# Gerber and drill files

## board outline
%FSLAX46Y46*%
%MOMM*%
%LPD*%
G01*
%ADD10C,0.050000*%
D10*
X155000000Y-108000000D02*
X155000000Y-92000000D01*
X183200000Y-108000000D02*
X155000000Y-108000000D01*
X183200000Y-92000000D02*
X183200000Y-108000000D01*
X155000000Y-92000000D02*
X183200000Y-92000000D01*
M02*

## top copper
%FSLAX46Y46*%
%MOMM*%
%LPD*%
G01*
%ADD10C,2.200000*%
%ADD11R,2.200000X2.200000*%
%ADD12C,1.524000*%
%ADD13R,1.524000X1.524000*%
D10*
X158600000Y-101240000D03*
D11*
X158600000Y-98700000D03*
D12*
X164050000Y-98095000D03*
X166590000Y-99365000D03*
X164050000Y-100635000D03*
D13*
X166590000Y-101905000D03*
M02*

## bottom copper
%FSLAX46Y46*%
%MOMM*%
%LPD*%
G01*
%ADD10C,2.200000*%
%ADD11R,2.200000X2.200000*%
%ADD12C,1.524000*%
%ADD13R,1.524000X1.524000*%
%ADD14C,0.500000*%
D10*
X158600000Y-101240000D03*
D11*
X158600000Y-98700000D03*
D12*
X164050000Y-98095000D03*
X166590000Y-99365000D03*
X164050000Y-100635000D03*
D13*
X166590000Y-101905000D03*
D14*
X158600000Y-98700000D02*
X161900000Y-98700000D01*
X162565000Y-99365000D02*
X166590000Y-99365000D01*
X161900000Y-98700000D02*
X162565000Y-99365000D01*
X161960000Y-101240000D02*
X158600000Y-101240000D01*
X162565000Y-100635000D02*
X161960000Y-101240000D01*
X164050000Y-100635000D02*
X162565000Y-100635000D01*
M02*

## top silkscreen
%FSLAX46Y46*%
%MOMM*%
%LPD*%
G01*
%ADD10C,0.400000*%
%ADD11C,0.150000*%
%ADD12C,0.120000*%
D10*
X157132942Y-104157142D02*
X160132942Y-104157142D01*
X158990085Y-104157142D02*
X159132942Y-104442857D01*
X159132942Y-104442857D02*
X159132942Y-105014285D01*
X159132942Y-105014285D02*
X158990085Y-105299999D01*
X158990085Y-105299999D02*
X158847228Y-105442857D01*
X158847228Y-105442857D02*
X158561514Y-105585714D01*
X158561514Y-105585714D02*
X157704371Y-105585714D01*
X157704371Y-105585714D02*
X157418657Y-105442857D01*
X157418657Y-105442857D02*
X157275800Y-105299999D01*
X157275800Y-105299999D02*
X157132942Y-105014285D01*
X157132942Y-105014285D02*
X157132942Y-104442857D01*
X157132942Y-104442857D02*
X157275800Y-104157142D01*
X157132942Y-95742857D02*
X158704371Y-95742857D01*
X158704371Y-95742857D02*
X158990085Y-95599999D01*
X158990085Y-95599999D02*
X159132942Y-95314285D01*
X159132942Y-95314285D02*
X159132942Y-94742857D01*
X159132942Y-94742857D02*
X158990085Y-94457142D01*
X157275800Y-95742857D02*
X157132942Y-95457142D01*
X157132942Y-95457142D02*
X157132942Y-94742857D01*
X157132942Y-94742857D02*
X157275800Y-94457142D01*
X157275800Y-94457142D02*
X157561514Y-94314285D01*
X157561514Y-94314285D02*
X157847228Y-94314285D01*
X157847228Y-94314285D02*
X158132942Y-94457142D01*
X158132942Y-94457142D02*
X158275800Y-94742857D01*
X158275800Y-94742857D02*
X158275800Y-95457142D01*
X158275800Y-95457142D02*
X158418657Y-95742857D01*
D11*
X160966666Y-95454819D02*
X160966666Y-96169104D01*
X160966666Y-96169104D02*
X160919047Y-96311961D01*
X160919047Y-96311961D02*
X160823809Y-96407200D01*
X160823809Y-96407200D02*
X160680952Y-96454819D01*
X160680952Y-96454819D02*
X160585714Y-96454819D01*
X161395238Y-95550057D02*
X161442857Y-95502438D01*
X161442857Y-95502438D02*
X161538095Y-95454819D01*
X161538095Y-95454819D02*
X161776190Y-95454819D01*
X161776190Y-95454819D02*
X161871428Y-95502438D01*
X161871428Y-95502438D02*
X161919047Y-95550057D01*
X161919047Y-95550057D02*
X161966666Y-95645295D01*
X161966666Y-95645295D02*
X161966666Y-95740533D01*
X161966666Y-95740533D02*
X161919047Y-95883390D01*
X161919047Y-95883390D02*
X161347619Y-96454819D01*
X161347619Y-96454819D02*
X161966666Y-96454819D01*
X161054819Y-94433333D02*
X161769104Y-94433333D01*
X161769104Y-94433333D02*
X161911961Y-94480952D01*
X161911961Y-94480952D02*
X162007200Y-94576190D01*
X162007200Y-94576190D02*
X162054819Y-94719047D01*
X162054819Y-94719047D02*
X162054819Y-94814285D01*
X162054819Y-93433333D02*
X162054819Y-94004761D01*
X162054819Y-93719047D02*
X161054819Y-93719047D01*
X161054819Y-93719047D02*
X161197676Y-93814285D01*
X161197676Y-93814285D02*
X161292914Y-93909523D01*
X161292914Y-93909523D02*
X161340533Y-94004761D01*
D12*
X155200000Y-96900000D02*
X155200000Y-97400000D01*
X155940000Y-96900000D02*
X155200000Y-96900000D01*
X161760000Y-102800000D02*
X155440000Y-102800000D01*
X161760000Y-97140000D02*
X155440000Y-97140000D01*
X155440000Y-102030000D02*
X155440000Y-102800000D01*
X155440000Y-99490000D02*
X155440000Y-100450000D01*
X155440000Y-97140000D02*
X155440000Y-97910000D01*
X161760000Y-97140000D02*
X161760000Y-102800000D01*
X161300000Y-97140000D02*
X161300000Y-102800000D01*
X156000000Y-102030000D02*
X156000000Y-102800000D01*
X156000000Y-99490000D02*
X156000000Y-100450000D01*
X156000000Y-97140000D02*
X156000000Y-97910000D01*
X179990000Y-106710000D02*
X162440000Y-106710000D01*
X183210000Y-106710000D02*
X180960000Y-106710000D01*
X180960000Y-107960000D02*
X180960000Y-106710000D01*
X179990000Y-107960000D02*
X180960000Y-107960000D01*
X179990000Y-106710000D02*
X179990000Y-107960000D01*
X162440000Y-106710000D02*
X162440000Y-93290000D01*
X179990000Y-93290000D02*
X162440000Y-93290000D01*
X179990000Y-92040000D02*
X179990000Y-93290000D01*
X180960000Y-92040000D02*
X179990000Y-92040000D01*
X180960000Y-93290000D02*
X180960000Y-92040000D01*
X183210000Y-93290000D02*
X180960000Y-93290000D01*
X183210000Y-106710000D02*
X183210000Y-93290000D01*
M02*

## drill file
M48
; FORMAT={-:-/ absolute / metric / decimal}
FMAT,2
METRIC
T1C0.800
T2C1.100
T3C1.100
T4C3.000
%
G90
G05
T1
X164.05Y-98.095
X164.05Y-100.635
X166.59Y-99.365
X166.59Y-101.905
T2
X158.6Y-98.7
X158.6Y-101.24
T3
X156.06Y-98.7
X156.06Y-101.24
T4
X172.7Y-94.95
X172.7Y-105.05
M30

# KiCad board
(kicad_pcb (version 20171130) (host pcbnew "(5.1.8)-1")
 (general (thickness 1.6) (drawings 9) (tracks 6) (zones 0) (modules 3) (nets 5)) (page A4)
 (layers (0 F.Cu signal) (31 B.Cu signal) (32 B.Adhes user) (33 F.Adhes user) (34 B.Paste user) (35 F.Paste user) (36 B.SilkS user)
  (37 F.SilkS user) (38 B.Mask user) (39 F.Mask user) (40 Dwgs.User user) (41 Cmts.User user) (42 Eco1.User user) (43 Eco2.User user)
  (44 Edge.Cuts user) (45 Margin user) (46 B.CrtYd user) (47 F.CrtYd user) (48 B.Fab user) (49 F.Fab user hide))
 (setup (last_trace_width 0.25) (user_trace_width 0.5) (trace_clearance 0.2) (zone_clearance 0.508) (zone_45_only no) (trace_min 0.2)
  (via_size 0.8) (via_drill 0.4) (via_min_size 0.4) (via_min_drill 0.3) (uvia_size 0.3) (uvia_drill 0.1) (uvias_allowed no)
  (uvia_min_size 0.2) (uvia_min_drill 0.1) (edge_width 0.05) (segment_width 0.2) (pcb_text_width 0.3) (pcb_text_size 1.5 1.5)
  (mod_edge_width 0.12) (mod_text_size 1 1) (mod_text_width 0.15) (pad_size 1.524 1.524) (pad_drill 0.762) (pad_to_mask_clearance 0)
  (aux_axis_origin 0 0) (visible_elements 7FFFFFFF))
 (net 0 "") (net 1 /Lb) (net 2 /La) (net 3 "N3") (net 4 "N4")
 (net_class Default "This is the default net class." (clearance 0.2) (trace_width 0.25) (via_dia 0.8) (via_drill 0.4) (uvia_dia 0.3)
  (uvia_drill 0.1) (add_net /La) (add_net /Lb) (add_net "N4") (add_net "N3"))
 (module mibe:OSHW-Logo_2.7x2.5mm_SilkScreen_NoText (layer B.Cu) (at 172.7 100 270)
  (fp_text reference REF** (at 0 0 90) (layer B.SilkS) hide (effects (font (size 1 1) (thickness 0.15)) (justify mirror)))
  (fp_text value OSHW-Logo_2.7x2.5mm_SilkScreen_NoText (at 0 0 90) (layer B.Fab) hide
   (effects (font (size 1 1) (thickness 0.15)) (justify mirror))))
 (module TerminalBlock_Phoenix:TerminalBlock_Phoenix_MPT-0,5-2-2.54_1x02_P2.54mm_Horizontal (layer F.Cu) (at 158.6 98.7 270)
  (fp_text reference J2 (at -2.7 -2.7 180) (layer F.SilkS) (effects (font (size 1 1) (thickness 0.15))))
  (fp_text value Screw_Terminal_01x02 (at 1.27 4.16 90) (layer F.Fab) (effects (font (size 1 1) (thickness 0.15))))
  (fp_line (start -1.8 3.4) (end -1.3 3.4) (layer F.SilkS) (width 0.12))
  (fp_line (start -1.8 2.66) (end -1.8 3.4) (layer F.SilkS) (width 0.12))
  (fp_line (start 4.1 -3.16) (end 4.1 3.16) (layer F.SilkS) (width 0.12))
  (fp_line (start -1.56 -3.16) (end -1.56 3.16) (layer F.SilkS) (width 0.12))
  (fp_line (start 3.33 3.16) (end 4.1 3.16) (layer F.SilkS) (width 0.12))
  (fp_line (start 0.79 3.16) (end 1.75 3.16) (layer F.SilkS) (width 0.12))
  (fp_line (start -1.56 3.16) (end -0.79 3.16) (layer F.SilkS) (width 0.12))
  (fp_line (start -1.56 -3.16) (end 4.1 -3.16) (layer F.SilkS) (width 0.12))
  (fp_line (start -1.56 -2.7) (end 4.1 -2.7) (layer F.SilkS) (width 0.12))
  (fp_line (start 3.33 2.6) (end 4.1 2.6) (layer F.SilkS) (width 0.12))
  (fp_line (start 0.79 2.6) (end 1.75 2.6) (layer F.SilkS) (width 0.12))
  (fp_line (start -1.56 2.6) (end -0.79 2.6) (layer F.SilkS) (width 0.12))
  (pad "" np_thru_hole circle (at 2.54 2.54 270) (size 1.1 1.1) (drill 1.1) (layers *.Cu *.Mask))
  (pad 2 thru_hole circle (at 2.54 0 270) (size 2.2 2.2) (drill 1.1) (layers *.Cu *.Mask) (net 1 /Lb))
  (pad "" np_thru_hole circle (at 0 2.54 270) (size 1.1 1.1) (drill 1.1) (layers *.Cu *.Mask))
  (pad 1 thru_hole rect (at 0 0 270) (size 2.2 2.2) (drill 1.1) (layers *.Cu *.Mask) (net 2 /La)))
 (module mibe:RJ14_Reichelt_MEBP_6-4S (layer F.Cu) (at 183.1 100 90)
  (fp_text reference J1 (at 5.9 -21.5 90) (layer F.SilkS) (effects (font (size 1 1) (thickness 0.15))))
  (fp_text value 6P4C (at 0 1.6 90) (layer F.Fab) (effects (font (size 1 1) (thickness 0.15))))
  (fp_line (start -6.71 -3.11) (end -6.71 -20.66) (layer F.SilkS) (width 0.12))
  (fp_line (start -6.71 0.11) (end -6.71 -2.14) (layer F.SilkS) (width 0.12))
  (fp_line (start -7.96 -2.14) (end -6.71 -2.14) (layer F.SilkS) (width 0.12))
  (fp_line (start -7.96 -3.11) (end -7.96 -2.14) (layer F.SilkS) (width 0.12))
  (fp_line (start -6.71 -3.11) (end -7.96 -3.11) (layer F.SilkS) (width 0.12))
  (fp_line (start -6.71 -20.66) (end 6.71 -20.66) (layer F.SilkS) (width 0.12))
  (fp_line (start 6.71 -3.11) (end 6.71 -20.66) (layer F.SilkS) (width 0.12))
  (fp_line (start 7.96 -3.11) (end 6.71 -3.11) (layer F.SilkS) (width 0.12))
  (fp_line (start 7.96 -2.14) (end 7.96 -3.11) (layer F.SilkS) (width 0.12))
  (fp_line (start 6.71 -2.14) (end 7.96 -2.14) (layer F.SilkS) (width 0.12))
  (fp_line (start 6.71 0.11) (end 6.71 -2.14) (layer F.SilkS) (width 0.12))
  (fp_line (start -6.71 0.11) (end 6.71 0.11) (layer F.SilkS) (width 0.12))
  (pad "" np_thru_hole circle (at 5.05 -10.4 90) (size 3 3) (drill 3) (layers *.Cu *.Mask))
  (pad "" np_thru_hole circle (at -5.05 -10.4 90) (size 3 3) (drill 3) (layers *.Cu *.Mask))
  (pad 4 thru_hole circle (at 1.905 -19.05 90) (size 1.524 1.524) (drill 0.8) (layers *.Cu *.Mask) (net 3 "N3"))
  (pad 3 thru_hole circle (at 0.635 -16.51 90) (size 1.524 1.524) (drill 0.8) (layers *.Cu *.Mask) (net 2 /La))
  (pad 2 thru_hole circle (at -0.635 -19.05 90) (size 1.524 1.524) (drill 0.8) (layers *.Cu *.Mask) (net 1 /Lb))
  (pad 1 thru_hole rect (at -1.905 -16.51 90) (size 1.524 1.524) (drill 0.8) (layers *.Cu *.Mask) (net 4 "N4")))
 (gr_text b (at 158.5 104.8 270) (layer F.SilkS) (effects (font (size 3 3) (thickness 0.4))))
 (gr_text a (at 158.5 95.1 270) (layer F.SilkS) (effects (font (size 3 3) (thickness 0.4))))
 (gr_line (start 155 108) (end 155 92) (layer Edge.Cuts) (width 0.05))
 (gr_line (start 183.2 108) (end 155 108) (layer Edge.Cuts) (width 0.05))
 (gr_line (start 183.2 92) (end 183.2 108) (layer Edge.Cuts) (width 0.05))
 (gr_line (start 155 92) (end 183.2 92) (layer Edge.Cuts) (width 0.05))
 (segment (start 158.6 98.7) (end 161.9 98.7) (width 0.5) (layer B.Cu) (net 2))
 (segment (start 162.565 99.365) (end 166.59 99.365) (width 0.5) (layer B.Cu) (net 2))
 (segment (start 161.9 98.7) (end 162.565 99.365) (width 0.5) (layer B.Cu) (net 2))
 (segment (start 161.96 101.24) (end 158.6 101.24) (width 0.5) (layer B.Cu) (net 1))
 (segment (start 162.565 100.635) (end 161.96 101.24) (width 0.5) (layer B.Cu) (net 1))
 (segment (start 164.05 100.635) (end 162.565 100.635) (width 0.5) (layer B.Cu) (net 1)))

